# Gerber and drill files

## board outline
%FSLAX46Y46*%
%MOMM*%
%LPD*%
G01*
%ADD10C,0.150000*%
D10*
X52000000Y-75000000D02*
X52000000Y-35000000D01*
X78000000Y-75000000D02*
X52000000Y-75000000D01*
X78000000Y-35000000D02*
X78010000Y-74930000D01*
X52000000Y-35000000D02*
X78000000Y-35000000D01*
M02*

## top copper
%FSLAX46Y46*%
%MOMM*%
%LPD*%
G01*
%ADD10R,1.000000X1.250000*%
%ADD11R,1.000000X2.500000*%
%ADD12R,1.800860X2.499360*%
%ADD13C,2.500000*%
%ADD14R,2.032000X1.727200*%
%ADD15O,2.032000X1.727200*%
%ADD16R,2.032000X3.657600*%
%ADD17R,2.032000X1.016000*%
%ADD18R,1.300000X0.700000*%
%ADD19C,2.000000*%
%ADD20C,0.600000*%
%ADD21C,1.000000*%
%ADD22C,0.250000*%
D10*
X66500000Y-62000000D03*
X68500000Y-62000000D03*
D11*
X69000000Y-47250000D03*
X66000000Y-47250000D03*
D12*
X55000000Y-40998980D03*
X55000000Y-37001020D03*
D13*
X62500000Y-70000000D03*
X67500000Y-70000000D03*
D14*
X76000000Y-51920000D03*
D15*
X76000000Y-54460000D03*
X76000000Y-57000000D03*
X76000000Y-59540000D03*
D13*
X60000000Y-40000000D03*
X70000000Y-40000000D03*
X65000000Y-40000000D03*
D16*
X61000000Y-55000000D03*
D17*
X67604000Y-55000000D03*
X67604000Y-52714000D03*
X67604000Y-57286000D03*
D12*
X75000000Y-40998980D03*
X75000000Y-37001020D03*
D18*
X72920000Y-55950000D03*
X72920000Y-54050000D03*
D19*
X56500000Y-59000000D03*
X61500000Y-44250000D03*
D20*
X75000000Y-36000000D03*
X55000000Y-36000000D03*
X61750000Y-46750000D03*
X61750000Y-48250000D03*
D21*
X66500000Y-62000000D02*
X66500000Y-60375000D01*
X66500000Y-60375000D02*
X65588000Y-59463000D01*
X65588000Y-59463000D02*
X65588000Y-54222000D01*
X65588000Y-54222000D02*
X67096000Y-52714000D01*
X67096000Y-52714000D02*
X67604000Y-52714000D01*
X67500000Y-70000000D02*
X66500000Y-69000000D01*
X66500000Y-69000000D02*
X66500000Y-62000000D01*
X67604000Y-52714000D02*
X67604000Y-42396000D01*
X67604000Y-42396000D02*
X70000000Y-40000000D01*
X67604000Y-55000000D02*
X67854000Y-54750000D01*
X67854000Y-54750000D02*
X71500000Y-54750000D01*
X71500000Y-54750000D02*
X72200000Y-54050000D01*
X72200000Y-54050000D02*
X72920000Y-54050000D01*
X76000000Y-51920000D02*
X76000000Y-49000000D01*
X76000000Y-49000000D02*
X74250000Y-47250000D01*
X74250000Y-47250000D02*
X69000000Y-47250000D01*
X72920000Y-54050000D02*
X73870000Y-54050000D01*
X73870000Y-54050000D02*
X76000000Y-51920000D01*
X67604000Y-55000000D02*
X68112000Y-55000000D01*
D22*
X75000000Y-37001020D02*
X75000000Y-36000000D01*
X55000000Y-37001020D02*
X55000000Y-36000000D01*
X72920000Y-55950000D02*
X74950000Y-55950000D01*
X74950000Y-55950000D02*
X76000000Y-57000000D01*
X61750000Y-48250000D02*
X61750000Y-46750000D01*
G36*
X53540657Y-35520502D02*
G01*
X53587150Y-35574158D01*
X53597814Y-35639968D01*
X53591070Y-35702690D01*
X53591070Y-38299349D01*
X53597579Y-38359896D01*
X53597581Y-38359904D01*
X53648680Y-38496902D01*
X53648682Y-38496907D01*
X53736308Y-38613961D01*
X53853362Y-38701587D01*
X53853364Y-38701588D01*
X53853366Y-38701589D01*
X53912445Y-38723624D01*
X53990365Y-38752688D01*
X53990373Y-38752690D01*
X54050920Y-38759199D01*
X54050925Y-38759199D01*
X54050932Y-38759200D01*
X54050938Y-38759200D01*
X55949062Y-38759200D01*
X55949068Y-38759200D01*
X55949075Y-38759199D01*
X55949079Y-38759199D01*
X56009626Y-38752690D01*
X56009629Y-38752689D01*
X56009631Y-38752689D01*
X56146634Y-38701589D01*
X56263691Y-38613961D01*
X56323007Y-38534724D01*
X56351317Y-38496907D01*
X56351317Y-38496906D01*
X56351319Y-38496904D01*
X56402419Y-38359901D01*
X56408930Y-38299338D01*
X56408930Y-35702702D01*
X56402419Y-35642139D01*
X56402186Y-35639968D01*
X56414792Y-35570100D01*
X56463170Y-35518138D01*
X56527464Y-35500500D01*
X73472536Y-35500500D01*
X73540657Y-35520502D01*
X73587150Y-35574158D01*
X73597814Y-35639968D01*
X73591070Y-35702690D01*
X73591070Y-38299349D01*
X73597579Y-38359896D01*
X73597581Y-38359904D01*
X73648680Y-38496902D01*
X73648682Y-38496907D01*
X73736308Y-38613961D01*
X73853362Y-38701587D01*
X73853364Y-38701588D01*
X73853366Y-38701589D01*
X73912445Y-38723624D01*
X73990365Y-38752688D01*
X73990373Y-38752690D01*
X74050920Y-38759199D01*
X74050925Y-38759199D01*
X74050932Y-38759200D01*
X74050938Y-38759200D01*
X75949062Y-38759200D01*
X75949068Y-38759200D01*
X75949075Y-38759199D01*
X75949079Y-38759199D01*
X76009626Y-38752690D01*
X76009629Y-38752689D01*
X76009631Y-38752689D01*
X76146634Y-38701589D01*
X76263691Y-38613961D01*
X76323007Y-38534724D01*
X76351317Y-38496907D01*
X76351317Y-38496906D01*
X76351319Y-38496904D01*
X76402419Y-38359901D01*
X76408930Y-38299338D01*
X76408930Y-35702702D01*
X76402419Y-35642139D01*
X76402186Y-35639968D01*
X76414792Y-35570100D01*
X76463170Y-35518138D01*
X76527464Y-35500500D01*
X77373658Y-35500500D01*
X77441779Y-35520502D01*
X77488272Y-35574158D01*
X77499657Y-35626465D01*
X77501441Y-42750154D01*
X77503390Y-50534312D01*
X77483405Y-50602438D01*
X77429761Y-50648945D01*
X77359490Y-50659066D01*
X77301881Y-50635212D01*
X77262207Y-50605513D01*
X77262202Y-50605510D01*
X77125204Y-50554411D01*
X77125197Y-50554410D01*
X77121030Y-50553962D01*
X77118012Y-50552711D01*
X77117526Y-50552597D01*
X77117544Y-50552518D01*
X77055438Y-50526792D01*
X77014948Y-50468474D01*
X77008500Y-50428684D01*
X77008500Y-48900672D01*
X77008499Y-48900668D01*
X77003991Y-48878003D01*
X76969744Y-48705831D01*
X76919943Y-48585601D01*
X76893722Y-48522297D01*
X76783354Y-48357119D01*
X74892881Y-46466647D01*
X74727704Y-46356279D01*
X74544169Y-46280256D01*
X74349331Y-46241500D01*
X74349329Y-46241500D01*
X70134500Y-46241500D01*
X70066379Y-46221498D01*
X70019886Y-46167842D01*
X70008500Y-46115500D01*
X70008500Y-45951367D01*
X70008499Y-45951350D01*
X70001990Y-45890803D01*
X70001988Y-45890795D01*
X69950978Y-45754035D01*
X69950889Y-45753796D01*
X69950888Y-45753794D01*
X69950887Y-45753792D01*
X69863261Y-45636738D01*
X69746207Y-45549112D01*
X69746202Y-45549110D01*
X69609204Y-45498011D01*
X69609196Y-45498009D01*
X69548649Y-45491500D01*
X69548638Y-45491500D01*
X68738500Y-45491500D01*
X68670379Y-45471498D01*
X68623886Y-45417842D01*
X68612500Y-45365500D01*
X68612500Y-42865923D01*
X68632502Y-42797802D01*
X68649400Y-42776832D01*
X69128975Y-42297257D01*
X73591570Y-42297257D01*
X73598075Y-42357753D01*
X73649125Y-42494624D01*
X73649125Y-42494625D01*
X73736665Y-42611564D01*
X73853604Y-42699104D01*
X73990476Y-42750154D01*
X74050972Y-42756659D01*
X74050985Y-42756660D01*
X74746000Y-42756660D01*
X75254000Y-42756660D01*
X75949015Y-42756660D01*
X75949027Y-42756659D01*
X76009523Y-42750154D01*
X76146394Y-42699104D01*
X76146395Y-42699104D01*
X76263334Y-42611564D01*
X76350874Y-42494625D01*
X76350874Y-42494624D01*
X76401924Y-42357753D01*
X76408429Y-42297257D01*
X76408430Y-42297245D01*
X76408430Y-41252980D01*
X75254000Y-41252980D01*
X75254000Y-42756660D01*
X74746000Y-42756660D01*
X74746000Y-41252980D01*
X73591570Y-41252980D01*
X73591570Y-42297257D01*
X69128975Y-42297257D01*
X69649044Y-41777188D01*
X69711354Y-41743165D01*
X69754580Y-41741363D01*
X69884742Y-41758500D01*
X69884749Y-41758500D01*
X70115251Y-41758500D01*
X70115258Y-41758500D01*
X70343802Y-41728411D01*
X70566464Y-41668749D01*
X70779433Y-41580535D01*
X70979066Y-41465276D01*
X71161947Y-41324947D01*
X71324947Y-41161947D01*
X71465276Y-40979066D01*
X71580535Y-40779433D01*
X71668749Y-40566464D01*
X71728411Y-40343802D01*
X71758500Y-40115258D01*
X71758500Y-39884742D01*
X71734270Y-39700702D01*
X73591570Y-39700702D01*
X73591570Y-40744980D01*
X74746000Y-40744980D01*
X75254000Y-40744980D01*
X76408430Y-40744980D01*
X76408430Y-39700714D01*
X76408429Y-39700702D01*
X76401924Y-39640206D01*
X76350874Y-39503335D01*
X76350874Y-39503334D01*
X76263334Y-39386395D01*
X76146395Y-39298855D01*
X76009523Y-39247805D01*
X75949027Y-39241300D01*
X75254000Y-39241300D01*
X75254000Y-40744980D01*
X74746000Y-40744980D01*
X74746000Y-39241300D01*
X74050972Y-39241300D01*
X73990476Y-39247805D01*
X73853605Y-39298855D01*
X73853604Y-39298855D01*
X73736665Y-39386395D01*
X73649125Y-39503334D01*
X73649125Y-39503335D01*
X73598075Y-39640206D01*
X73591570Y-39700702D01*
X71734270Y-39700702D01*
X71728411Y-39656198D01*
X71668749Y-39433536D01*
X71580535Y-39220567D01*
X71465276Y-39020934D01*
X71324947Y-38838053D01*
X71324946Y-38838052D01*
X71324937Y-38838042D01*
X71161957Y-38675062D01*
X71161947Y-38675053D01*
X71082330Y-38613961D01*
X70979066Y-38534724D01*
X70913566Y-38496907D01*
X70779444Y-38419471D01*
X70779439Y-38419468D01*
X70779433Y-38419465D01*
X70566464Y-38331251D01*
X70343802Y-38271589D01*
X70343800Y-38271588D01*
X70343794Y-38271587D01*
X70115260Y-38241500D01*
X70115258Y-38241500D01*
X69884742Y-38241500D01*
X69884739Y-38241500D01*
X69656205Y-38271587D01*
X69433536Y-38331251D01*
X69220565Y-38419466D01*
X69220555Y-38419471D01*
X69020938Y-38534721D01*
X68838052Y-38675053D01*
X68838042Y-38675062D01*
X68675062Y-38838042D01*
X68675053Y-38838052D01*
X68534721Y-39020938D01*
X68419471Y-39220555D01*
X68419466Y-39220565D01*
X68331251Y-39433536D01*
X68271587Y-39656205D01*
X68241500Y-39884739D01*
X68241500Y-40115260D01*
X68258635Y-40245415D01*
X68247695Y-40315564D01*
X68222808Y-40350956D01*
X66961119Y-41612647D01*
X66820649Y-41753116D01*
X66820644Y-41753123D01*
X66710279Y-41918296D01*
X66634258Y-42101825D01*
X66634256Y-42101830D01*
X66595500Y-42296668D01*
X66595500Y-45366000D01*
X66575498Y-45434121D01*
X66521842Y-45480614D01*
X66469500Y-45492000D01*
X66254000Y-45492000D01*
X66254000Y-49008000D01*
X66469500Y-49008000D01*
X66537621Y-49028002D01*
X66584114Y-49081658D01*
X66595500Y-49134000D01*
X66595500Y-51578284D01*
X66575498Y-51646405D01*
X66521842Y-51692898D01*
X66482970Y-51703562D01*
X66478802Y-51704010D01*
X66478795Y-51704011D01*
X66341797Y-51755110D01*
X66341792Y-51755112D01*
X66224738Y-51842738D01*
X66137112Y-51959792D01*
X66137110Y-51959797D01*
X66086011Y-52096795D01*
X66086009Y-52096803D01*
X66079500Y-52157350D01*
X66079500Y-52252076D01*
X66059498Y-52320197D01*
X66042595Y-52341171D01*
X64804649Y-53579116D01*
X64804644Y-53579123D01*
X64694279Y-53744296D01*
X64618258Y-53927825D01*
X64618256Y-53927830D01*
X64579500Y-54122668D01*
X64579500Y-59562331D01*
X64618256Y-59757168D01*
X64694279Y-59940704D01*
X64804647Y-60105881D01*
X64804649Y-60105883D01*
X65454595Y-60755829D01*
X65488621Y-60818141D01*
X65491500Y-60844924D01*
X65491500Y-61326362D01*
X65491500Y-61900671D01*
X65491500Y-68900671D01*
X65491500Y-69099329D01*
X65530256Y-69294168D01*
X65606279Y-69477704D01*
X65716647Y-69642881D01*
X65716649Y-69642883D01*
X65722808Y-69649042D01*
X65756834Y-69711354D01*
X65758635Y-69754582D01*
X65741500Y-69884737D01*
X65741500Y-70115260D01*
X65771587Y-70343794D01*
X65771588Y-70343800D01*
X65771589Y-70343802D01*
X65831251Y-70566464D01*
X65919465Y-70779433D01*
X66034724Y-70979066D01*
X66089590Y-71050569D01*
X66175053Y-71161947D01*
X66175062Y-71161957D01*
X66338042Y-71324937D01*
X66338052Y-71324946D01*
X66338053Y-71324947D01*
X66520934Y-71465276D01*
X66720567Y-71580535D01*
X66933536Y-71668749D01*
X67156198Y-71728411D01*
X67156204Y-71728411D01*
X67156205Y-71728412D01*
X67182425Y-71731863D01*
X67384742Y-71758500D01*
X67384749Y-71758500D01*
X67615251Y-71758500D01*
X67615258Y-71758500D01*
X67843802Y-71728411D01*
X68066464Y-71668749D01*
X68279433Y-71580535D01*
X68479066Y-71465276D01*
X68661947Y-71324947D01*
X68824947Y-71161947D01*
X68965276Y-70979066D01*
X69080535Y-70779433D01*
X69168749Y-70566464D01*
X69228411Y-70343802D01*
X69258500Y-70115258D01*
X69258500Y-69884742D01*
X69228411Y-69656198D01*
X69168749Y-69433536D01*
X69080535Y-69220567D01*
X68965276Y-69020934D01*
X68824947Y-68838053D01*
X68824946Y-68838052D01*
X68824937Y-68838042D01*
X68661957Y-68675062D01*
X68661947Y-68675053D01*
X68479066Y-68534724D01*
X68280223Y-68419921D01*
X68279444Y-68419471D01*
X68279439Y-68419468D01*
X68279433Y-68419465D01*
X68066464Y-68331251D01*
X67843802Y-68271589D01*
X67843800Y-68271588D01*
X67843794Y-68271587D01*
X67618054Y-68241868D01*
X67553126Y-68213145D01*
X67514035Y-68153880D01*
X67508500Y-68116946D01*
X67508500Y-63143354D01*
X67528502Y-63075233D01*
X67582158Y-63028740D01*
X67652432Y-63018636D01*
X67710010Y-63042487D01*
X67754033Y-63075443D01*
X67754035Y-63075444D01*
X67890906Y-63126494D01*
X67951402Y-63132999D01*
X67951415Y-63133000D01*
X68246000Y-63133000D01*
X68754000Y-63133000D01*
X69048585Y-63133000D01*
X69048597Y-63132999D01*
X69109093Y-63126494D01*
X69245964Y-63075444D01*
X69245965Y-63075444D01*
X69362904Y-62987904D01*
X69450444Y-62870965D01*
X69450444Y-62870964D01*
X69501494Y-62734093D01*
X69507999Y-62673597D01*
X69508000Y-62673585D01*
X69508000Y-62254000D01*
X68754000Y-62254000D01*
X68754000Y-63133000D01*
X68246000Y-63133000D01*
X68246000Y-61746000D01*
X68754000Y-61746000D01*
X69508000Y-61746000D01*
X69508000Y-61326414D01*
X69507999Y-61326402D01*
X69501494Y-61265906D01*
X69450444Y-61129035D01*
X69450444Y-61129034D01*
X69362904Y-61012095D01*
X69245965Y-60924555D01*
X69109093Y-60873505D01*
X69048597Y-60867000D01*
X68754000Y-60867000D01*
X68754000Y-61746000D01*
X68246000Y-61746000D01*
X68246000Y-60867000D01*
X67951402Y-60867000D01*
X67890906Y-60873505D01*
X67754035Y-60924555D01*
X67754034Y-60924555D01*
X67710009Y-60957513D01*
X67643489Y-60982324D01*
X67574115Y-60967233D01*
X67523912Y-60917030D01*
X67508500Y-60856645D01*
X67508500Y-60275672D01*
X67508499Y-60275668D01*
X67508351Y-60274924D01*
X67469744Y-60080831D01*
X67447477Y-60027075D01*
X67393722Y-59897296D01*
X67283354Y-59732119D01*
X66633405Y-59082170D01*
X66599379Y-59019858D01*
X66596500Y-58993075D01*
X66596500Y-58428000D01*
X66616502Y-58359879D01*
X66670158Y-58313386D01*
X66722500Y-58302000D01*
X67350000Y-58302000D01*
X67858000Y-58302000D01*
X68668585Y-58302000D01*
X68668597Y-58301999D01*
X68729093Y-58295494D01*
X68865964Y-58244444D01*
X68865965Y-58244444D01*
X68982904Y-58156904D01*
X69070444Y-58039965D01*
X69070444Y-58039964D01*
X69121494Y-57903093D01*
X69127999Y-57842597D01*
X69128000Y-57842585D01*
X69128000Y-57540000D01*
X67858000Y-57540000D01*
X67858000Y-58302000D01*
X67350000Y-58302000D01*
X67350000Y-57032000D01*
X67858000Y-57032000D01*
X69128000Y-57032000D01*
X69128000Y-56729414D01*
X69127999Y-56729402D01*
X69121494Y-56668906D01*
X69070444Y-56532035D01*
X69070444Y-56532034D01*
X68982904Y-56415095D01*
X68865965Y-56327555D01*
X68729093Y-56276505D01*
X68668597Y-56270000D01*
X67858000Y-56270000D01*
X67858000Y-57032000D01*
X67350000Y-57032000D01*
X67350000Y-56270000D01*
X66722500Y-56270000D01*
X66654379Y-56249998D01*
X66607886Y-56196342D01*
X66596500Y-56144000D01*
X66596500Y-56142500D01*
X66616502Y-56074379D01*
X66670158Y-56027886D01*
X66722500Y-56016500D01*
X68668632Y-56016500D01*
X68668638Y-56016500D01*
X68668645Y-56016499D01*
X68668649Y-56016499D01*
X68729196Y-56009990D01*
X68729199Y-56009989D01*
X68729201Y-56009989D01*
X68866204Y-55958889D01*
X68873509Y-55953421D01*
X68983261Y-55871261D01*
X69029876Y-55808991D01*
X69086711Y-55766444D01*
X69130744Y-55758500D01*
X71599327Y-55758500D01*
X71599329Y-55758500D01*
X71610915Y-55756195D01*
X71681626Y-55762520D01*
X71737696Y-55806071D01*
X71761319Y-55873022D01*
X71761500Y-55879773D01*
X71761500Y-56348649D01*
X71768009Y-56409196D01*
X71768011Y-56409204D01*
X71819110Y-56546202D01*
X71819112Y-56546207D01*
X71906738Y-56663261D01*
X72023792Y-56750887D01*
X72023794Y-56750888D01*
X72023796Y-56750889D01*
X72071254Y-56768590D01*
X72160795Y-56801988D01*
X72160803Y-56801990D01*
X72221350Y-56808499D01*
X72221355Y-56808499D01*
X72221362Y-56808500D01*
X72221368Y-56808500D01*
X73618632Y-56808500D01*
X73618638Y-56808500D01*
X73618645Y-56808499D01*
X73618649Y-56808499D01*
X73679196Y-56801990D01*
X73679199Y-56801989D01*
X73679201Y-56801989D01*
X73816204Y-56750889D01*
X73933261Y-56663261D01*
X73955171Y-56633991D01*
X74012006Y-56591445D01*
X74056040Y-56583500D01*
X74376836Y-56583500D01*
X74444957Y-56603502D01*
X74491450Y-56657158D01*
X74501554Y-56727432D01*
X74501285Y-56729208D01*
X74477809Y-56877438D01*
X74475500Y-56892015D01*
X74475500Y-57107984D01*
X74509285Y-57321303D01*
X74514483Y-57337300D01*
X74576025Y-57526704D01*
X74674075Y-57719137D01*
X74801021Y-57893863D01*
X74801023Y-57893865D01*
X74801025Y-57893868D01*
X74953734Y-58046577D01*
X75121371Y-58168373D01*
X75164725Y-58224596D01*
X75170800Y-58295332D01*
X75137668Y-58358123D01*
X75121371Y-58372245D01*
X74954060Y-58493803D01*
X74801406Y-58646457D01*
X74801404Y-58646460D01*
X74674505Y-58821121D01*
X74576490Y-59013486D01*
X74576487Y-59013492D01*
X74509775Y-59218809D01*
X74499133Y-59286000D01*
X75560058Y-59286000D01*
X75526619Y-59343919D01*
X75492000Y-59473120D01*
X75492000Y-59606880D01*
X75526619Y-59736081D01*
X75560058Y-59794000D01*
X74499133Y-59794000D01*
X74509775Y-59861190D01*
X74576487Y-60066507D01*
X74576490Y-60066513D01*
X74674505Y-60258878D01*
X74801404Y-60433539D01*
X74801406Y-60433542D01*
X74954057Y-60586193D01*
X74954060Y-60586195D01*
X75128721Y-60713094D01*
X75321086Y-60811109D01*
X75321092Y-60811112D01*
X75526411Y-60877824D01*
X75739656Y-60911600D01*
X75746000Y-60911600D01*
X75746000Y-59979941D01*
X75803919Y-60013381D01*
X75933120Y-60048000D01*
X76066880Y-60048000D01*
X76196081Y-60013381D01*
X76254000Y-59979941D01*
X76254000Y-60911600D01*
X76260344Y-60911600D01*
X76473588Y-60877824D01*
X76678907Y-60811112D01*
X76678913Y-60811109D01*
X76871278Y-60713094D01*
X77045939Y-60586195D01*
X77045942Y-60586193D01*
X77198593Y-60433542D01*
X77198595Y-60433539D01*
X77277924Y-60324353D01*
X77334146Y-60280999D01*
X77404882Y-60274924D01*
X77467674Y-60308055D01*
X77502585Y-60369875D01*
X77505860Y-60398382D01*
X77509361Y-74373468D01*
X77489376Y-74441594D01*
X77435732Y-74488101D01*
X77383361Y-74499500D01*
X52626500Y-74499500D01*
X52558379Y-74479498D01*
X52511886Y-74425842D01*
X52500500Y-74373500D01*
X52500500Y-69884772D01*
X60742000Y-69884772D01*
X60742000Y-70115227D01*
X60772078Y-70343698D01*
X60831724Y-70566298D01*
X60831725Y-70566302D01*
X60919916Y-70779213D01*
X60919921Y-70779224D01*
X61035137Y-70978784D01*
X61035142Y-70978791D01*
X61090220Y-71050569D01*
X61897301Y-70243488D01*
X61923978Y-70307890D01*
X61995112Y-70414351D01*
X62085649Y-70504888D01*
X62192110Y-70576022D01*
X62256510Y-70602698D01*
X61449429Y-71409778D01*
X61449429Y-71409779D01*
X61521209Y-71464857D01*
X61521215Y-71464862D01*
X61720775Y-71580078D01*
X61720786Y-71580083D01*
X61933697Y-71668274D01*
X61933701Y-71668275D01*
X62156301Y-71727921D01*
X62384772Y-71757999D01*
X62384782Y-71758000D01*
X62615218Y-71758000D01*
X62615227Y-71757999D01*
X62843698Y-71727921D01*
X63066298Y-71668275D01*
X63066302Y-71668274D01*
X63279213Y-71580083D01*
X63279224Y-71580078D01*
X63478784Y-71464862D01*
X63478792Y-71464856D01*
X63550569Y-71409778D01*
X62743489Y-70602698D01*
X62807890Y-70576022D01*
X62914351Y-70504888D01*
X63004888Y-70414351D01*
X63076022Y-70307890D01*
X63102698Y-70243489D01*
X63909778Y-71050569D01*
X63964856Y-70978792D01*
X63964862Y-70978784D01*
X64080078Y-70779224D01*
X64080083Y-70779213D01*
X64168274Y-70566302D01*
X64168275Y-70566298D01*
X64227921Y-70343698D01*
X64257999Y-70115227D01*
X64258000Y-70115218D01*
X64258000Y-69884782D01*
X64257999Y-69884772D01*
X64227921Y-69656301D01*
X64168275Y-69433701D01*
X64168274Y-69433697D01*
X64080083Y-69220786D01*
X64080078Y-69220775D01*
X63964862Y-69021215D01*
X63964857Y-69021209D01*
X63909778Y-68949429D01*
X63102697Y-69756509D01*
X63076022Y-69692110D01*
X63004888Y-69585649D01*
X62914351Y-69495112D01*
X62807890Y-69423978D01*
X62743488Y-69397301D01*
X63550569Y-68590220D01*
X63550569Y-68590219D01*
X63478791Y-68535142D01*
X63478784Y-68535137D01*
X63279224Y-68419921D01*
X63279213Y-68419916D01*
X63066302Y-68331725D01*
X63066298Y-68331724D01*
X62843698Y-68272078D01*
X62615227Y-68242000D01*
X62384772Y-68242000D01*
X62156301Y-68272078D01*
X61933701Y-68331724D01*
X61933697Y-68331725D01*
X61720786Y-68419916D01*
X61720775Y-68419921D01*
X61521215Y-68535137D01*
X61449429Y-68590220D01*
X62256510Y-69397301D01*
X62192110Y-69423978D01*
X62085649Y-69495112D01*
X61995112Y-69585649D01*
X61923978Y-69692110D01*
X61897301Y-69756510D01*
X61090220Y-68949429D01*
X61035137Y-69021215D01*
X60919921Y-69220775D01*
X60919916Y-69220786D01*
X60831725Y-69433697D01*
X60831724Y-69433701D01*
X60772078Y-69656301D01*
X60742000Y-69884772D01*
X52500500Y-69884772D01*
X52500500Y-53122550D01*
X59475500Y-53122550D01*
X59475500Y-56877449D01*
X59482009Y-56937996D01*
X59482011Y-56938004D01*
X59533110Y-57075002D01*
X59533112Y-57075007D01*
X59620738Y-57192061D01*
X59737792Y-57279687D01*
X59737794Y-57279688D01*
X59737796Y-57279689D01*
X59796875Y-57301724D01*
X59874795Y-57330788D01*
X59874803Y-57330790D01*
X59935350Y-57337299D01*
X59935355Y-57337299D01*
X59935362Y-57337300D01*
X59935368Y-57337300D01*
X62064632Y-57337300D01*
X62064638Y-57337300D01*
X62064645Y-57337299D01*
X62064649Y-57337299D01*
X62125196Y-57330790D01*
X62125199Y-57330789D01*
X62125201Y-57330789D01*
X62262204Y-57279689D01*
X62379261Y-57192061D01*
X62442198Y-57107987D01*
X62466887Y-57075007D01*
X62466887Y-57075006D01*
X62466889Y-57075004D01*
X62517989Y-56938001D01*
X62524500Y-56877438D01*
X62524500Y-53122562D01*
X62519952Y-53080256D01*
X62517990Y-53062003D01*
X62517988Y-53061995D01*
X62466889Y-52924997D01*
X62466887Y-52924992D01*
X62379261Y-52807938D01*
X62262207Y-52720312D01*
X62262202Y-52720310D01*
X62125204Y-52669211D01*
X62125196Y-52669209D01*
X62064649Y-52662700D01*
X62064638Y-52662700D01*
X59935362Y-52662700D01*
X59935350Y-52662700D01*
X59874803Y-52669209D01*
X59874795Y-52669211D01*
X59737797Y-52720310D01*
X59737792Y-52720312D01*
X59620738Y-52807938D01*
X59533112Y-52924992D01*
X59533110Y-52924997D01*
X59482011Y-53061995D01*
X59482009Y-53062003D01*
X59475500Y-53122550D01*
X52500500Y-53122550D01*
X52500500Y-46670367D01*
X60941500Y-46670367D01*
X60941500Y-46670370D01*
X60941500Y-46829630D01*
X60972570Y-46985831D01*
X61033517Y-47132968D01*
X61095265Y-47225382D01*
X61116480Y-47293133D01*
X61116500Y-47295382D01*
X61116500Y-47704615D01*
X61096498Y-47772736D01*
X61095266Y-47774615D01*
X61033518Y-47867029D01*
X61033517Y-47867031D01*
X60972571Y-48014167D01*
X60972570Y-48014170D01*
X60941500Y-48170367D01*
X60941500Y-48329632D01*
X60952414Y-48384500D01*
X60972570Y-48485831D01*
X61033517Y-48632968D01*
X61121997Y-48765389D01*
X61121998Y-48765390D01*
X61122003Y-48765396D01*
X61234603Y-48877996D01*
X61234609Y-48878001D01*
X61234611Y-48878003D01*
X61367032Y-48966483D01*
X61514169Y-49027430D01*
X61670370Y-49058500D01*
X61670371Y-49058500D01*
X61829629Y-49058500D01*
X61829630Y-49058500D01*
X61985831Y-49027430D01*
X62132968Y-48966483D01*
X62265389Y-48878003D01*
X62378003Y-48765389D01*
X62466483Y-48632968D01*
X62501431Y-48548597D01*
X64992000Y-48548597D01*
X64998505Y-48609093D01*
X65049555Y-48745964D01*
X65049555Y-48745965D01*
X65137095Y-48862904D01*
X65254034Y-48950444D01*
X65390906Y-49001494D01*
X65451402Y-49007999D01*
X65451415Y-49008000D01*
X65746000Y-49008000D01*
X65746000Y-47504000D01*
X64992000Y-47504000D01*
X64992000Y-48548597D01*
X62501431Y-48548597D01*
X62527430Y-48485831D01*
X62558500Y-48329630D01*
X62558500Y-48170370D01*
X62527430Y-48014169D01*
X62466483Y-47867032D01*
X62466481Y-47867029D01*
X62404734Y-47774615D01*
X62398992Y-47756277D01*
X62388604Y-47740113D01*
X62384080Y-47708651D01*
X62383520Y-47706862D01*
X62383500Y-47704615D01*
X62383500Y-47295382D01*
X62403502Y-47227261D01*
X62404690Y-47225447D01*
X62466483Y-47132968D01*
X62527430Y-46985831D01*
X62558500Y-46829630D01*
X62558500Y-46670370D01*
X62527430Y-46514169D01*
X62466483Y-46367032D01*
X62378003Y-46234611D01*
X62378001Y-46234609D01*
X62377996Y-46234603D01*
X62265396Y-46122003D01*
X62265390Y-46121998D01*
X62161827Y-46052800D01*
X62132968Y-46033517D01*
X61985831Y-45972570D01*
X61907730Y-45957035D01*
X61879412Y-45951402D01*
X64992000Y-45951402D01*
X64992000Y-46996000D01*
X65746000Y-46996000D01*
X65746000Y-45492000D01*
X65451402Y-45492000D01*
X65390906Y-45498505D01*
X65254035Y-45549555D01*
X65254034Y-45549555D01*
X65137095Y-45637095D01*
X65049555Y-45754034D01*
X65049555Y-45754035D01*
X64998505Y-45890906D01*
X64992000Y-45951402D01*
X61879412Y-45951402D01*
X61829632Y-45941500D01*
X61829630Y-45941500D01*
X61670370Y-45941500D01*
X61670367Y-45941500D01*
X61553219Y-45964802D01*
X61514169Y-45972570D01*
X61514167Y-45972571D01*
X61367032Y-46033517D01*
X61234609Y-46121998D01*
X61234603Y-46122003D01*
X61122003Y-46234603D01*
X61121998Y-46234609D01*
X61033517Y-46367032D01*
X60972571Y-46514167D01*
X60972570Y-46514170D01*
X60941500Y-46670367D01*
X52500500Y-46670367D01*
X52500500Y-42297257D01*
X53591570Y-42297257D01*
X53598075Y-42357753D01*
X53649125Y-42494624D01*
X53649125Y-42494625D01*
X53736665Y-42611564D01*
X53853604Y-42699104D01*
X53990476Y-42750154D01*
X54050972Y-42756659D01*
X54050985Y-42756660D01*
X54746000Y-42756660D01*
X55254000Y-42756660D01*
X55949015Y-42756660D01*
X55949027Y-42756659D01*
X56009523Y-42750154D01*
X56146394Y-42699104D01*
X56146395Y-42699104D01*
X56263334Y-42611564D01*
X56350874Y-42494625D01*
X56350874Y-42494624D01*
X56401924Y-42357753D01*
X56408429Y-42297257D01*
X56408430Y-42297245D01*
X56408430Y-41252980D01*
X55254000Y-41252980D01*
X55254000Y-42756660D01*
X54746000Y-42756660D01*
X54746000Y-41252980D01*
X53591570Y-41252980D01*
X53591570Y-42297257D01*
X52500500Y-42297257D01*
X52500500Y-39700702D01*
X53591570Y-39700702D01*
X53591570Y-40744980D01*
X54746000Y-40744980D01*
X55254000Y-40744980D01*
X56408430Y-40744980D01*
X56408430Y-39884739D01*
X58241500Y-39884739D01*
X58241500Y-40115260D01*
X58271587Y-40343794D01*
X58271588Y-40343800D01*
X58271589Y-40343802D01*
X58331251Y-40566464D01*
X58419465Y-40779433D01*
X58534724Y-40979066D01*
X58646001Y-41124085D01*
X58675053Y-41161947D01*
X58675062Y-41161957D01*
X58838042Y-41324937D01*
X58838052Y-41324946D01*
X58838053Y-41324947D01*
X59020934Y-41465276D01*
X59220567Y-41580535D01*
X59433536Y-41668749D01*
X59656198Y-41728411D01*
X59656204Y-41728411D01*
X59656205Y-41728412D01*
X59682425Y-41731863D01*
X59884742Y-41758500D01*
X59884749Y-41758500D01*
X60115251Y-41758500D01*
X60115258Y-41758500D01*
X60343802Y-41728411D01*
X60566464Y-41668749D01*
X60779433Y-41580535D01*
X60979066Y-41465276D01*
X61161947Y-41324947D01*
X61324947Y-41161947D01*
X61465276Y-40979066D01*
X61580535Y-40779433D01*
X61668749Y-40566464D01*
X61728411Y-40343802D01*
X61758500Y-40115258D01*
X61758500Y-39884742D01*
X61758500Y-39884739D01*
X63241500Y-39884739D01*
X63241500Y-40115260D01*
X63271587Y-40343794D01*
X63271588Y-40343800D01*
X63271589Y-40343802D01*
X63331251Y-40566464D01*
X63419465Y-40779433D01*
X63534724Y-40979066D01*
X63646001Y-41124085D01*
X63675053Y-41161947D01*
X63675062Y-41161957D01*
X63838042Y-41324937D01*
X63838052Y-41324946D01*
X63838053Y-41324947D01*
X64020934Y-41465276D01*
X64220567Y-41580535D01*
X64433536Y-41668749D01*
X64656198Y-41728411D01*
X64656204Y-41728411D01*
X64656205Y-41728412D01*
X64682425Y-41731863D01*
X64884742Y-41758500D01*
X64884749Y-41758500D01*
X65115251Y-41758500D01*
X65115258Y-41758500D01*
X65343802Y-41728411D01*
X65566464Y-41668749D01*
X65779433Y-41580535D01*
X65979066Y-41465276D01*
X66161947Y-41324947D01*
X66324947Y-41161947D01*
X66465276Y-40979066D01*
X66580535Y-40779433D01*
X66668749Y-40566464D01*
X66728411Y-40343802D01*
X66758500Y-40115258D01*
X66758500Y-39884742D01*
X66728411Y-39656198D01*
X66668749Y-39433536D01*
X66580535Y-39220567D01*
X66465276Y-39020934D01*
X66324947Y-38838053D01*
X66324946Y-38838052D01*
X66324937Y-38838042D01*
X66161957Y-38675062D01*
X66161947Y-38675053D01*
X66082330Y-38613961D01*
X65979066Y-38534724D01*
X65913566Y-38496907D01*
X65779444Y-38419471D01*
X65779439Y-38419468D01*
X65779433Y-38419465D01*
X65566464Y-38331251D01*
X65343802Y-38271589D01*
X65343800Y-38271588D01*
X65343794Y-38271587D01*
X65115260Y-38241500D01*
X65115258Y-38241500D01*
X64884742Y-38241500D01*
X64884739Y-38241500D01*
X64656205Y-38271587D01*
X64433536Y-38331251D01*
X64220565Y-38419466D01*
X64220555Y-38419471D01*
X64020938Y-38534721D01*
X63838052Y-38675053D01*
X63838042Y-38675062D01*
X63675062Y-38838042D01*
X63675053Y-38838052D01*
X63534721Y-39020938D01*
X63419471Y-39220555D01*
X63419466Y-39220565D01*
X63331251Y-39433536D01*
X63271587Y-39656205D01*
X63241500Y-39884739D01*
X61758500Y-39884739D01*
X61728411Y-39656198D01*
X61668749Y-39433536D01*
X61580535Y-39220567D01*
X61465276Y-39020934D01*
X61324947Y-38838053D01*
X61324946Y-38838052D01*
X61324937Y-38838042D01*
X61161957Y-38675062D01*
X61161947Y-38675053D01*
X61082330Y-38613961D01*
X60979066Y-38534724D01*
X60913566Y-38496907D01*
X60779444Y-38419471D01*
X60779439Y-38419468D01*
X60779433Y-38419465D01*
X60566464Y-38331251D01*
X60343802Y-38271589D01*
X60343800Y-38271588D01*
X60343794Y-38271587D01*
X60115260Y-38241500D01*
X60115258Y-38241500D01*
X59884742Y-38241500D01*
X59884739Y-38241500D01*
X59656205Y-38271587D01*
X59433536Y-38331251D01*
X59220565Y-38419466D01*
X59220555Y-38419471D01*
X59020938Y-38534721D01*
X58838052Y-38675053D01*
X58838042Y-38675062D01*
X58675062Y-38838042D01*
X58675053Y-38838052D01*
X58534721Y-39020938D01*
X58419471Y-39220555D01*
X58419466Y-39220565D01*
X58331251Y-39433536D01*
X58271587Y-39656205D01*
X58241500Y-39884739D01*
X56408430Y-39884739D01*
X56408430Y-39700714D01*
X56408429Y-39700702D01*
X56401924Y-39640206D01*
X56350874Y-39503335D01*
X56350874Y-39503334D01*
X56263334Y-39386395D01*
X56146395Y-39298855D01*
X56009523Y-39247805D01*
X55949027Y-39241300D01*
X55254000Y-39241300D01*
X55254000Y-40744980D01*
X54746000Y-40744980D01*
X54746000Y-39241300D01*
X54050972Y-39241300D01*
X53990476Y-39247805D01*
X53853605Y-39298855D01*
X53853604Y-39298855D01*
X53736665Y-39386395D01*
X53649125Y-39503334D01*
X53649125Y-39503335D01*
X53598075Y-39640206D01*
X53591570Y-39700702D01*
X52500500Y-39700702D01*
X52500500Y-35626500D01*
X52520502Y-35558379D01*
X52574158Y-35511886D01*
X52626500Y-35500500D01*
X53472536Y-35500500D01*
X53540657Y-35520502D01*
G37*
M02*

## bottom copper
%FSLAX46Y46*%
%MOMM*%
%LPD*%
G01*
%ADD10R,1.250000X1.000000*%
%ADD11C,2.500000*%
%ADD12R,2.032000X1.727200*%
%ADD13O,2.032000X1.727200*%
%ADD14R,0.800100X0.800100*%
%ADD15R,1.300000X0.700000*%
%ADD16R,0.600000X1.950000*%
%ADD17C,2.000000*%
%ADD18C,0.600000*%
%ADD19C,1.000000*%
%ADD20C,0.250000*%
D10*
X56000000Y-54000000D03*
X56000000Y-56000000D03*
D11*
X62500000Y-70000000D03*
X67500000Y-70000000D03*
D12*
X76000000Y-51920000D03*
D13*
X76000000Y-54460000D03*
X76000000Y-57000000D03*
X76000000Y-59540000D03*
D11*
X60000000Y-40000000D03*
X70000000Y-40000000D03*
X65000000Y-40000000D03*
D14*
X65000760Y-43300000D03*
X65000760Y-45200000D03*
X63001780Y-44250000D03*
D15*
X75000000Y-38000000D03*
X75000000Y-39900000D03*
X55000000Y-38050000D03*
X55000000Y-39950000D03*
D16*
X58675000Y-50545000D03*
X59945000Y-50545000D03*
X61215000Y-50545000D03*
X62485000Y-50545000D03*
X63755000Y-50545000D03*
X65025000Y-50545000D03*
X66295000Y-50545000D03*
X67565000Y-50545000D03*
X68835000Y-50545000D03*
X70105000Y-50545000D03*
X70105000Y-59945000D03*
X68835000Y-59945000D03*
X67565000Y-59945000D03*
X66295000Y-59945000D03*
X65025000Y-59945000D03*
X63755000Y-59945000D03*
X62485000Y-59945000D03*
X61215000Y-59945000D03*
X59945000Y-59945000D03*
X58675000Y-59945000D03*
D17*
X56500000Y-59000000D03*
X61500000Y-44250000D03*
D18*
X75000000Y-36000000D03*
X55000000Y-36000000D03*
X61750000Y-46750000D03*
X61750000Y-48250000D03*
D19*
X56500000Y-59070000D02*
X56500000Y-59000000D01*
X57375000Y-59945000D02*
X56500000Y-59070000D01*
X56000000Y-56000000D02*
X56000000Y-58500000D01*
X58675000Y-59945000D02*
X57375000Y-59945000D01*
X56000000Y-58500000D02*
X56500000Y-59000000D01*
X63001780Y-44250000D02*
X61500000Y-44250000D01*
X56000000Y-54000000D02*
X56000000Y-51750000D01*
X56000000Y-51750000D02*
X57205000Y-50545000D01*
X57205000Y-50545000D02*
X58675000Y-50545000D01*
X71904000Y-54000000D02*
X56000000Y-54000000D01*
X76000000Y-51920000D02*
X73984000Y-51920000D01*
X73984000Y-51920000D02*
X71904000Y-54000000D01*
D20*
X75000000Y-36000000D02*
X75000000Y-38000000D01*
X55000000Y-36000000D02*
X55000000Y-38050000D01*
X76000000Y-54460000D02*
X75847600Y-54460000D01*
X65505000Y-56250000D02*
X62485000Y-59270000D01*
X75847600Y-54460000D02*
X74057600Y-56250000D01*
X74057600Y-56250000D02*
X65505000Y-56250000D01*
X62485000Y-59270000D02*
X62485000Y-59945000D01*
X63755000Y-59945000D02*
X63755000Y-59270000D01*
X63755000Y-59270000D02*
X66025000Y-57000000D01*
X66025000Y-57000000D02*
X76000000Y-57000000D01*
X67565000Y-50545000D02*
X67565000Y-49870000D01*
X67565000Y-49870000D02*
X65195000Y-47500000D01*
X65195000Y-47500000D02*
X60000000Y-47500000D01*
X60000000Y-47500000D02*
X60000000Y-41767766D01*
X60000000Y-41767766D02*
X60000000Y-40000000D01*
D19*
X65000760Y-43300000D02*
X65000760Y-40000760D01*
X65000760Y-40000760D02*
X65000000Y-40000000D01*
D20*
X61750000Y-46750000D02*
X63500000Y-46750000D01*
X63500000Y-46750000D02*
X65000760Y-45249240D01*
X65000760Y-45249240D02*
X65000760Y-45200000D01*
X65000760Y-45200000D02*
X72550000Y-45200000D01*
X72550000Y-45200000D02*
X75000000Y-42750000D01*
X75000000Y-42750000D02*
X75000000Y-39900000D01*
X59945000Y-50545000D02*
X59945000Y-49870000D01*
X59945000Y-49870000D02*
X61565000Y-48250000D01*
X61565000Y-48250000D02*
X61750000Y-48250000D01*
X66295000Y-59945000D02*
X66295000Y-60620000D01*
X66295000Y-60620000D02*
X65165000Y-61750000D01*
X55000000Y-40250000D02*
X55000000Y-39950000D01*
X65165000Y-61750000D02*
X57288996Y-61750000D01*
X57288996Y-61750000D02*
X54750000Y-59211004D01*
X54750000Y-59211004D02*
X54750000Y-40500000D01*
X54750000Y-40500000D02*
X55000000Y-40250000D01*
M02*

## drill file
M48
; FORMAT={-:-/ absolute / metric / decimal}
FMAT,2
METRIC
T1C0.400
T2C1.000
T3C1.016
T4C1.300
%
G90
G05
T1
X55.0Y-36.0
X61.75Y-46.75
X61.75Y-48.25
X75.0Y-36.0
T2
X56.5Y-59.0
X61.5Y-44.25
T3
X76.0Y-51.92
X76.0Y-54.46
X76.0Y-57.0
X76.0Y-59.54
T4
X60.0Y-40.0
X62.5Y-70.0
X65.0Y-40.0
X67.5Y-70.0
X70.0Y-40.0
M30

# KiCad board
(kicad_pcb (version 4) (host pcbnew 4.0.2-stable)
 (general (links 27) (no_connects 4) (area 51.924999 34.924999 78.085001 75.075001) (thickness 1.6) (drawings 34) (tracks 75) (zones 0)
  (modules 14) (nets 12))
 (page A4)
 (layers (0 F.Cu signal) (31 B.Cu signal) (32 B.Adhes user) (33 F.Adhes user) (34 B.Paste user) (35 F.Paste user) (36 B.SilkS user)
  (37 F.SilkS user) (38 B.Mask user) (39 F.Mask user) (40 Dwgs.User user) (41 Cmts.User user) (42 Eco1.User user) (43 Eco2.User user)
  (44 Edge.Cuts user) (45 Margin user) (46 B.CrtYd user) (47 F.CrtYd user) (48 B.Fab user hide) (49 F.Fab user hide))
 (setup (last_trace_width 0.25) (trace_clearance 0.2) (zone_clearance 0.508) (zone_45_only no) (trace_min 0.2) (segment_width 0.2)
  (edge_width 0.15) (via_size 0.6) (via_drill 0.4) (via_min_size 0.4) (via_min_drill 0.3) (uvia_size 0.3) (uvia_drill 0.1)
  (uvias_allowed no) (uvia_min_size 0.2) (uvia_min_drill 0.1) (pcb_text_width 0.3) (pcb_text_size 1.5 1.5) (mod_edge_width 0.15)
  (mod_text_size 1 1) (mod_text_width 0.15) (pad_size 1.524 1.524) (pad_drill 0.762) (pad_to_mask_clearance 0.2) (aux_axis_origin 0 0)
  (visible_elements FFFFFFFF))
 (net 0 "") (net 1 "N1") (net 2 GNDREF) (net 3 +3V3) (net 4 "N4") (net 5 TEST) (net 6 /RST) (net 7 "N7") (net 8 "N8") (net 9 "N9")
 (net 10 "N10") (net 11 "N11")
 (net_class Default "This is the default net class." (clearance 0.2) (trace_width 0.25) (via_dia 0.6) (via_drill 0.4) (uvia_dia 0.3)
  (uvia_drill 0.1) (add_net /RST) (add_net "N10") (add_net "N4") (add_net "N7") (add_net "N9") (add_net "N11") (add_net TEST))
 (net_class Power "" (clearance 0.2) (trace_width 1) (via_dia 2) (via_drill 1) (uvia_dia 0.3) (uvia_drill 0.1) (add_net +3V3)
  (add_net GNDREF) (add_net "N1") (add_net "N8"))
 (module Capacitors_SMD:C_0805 (layer F.Cu) (at 67.5 62)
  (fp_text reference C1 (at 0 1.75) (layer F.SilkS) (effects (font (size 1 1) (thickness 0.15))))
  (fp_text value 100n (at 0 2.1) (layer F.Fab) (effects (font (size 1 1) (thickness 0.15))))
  (pad 1 smd rect (at -1 0) (size 1 1.25) (layers F.Cu F.Paste F.Mask) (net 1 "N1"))
  (pad 2 smd rect (at 1 0) (size 1 1.25) (layers F.Cu F.Paste F.Mask) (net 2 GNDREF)))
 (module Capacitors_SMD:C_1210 (layer F.Cu) (at 67.5 47.25 180)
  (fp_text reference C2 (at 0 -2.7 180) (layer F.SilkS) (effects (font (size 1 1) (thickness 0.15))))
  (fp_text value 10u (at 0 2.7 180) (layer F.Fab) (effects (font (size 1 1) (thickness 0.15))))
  (pad 1 smd rect (at -1.5 0 180) (size 1 2.5) (layers F.Cu F.Paste F.Mask) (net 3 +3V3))
  (pad 2 smd rect (at 1.5 0 180) (size 1 2.5) (layers F.Cu F.Paste F.Mask) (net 2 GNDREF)))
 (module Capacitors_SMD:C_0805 (layer B.Cu) (at 56 55 270)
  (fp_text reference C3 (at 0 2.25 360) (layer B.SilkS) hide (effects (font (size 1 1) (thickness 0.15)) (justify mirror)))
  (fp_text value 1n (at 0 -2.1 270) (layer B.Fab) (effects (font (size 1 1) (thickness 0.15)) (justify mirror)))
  (pad 1 smd rect (at -1 0 270) (size 1 1.25) (layers B.Cu B.Paste B.Mask) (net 3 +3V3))
  (pad 2 smd rect (at 1 0 270) (size 1 1.25) (layers B.Cu B.Paste B.Mask) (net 2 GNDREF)))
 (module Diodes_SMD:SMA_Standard (layer F.Cu) (at 55 39 90)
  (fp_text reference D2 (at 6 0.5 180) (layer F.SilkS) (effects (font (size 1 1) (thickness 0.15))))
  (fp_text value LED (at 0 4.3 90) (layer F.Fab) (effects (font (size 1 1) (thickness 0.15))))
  (pad 1 smd rect (at -1.99898 0 90) (size 2.49936 1.80086) (layers F.Cu F.Paste F.Mask) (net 2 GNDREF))
  (pad 2 smd rect (at 1.99898 0 90) (size 2.49936 1.80086) (layers F.Cu F.Paste F.Mask) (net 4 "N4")))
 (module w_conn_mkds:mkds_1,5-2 (layer F.Cu) (at 65 70)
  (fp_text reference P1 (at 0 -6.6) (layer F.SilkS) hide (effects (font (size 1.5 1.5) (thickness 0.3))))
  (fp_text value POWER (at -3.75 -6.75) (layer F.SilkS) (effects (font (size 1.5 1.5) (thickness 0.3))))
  (pad 1 thru_hole circle (at -2.5 0) (size 2.5 2.5) (drill 1.3) (layers *.Cu *.Mask F.SilkS) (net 2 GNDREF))
  (pad 2 thru_hole circle (at 2.5 0) (size 2.5 2.5) (drill 1.3) (layers *.Cu *.Mask F.SilkS) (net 1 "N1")))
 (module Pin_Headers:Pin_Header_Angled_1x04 (layer F.Cu) (at 76 51.92)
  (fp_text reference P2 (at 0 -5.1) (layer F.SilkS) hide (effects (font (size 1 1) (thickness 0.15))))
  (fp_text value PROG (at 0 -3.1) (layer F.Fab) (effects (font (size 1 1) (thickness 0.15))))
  (pad 1 thru_hole rect (at 0 0) (size 2.032 1.7272) (drill 1.016) (layers *.Cu *.Mask F.SilkS) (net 3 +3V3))
  (pad 2 thru_hole oval (at 0 2.54) (size 2.032 1.7272) (drill 1.016) (layers *.Cu *.Mask F.SilkS) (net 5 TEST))
  (pad 3 thru_hole oval (at 0 5.08) (size 2.032 1.7272) (drill 1.016) (layers *.Cu *.Mask F.SilkS) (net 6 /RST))
  (pad 4 thru_hole oval (at 0 7.62) (size 2.032 1.7272) (drill 1.016) (layers *.Cu *.Mask F.SilkS) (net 2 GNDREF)))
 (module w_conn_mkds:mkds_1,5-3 (layer F.Cu) (at 65 40 180)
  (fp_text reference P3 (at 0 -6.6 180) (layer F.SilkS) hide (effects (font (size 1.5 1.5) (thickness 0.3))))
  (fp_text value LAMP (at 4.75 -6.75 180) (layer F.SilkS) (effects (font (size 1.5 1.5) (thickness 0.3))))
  (pad 3 thru_hole circle (at 5 0 180) (size 2.5 2.5) (drill 1.3) (layers *.Cu *.Mask F.SilkS) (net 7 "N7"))
  (pad 1 thru_hole circle (at -5 0 180) (size 2.5 2.5) (drill 1.3) (layers *.Cu *.Mask F.SilkS) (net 1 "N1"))
  (pad 2 thru_hole circle (at 0 0 180) (size 2.5 2.5) (drill 1.3) (layers *.Cu *.Mask F.SilkS) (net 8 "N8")))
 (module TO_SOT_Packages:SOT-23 (layer B.Cu) (at 64 44.25 270)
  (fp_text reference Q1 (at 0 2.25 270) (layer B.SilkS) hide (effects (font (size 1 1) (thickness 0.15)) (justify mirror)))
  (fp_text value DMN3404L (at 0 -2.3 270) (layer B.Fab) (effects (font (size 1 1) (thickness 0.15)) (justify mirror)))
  (pad 1 smd rect (at -0.95 -1.00076 270) (size 0.8001 0.8001) (layers B.Cu B.Paste B.Mask) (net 8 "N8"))
  (pad 2 smd rect (at 0.95 -1.00076 270) (size 0.8001 0.8001) (layers B.Cu B.Paste B.Mask) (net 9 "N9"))
  (pad 3 smd rect (at 0 0.99822 270) (size 0.8001 0.8001) (layers B.Cu B.Paste B.Mask) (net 2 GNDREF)))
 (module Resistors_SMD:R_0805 (layer B.Cu) (at 75 38.95 270)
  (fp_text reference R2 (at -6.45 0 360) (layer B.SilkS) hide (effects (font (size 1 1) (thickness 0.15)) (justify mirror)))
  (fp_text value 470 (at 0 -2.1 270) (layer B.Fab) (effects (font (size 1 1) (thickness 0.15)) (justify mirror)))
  (pad 1 smd rect (at -0.95 0 270) (size 0.7 1.3) (layers B.Cu B.Paste B.Mask) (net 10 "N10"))
  (pad 2 smd rect (at 0.95 0 270) (size 0.7 1.3) (layers B.Cu B.Paste B.Mask) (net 9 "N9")))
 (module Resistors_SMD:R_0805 (layer B.Cu) (at 55 39 270)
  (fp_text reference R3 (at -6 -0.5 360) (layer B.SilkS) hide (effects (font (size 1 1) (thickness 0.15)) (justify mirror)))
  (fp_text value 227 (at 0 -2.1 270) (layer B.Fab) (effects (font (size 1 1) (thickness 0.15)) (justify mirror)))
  (pad 1 smd rect (at -0.95 0 270) (size 0.7 1.3) (layers B.Cu B.Paste B.Mask) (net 4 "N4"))
  (pad 2 smd rect (at 0.95 0 270) (size 0.7 1.3) (layers B.Cu B.Paste B.Mask) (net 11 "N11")))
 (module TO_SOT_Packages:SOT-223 (layer F.Cu) (at 64.302 55 90)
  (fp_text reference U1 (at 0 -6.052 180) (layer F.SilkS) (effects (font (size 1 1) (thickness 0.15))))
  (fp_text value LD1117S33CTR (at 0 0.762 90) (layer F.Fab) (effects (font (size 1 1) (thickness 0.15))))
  (pad 4 smd rect (at 0 -3.302 90) (size 3.6576 2.032) (layers F.Cu F.Paste F.Mask))
  (pad 2 smd rect (at 0 3.302 90) (size 1.016 2.032) (layers F.Cu F.Paste F.Mask) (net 3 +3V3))
  (pad 3 smd rect (at 2.286 3.302 90) (size 1.016 2.032) (layers F.Cu F.Paste F.Mask) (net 1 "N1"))
  (pad 1 smd rect (at -2.286 3.302 90) (size 1.016 2.032) (layers F.Cu F.Paste F.Mask) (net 2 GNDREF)))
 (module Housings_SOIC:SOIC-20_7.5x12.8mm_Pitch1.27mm (layer B.Cu) (at 64.39 55.245 270)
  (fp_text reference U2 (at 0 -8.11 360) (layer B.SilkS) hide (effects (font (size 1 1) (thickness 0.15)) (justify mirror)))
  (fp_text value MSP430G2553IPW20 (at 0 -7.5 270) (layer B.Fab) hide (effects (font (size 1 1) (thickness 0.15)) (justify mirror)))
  (pad 1 smd rect (at -4.7 5.715 270) (size 1.95 0.6) (layers B.Cu B.Paste B.Mask) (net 3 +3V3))
  (pad 2 smd rect (at -4.7 4.445 270) (size 1.95 0.6) (layers B.Cu B.Paste B.Mask) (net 9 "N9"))
  (pad 3 smd rect (at -4.7 3.175 270) (size 1.95 0.6) (layers B.Cu B.Paste B.Mask))
  (pad 4 smd rect (at -4.7 1.905 270) (size 1.95 0.6) (layers B.Cu B.Paste B.Mask))
  (pad 5 smd rect (at -4.7 0.635 270) (size 1.95 0.6) (layers B.Cu B.Paste B.Mask))
  (pad 6 smd rect (at -4.7 -0.635 270) (size 1.95 0.6) (layers B.Cu B.Paste B.Mask))
  (pad 7 smd rect (at -4.7 -1.905 270) (size 1.95 0.6) (layers B.Cu B.Paste B.Mask))
  (pad 8 smd rect (at -4.7 -3.175 270) (size 1.95 0.6) (layers B.Cu B.Paste B.Mask) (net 7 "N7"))
  (pad 9 smd rect (at -4.7 -4.445 270) (size 1.95 0.6) (layers B.Cu B.Paste B.Mask))
  (pad 10 smd rect (at -4.7 -5.715 270) (size 1.95 0.6) (layers B.Cu B.Paste B.Mask))
  (pad 11 smd rect (at 4.7 -5.715 270) (size 1.95 0.6) (layers B.Cu B.Paste B.Mask))
  (pad 12 smd rect (at 4.7 -4.445 270) (size 1.95 0.6) (layers B.Cu B.Paste B.Mask))
  (pad 13 smd rect (at 4.7 -3.175 270) (size 1.95 0.6) (layers B.Cu B.Paste B.Mask))
  (pad 14 smd rect (at 4.7 -1.905 270) (size 1.95 0.6) (layers B.Cu B.Paste B.Mask) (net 11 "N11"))
  (pad 15 smd rect (at 4.7 -0.635 270) (size 1.95 0.6) (layers B.Cu B.Paste B.Mask))
  (pad 16 smd rect (at 4.7 0.635 270) (size 1.95 0.6) (layers B.Cu B.Paste B.Mask) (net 6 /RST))
  (pad 17 smd rect (at 4.7 1.905 270) (size 1.95 0.6) (layers B.Cu B.Paste B.Mask) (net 5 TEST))
  (pad 18 smd rect (at 4.7 3.175 270) (size 1.95 0.6) (layers B.Cu B.Paste B.Mask))
  (pad 19 smd rect (at 4.7 4.445 270) (size 1.95 0.6) (layers B.Cu B.Paste B.Mask))
  (pad 20 smd rect (at 4.7 5.715 270) (size 1.95 0.6) (layers B.Cu B.Paste B.Mask) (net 2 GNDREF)))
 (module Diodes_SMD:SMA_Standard (layer F.Cu) (at 75 39 90)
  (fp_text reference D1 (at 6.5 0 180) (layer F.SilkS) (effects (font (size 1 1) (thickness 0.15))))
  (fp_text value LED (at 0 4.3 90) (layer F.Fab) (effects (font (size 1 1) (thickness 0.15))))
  (pad 1 smd rect (at -1.99898 0 90) (size 2.49936 1.80086) (layers F.Cu F.Paste F.Mask) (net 2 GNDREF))
  (pad 2 smd rect (at 1.99898 0 90) (size 2.49936 1.80086) (layers F.Cu F.Paste F.Mask) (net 10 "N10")))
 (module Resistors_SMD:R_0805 (layer F.Cu) (at 72.92 55 90)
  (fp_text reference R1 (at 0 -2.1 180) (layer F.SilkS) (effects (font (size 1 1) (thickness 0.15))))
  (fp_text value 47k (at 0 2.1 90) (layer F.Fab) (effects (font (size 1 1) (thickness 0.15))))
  (pad 1 smd rect (at -0.95 0 90) (size 0.7 1.3) (layers F.Cu F.Paste F.Mask) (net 6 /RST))
  (pad 2 smd rect (at 0.95 0 90) (size 0.7 1.3) (layers F.Cu F.Paste F.Mask) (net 3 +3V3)))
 (gr_line (start 52 75) (end 52 35) (layer Edge.Cuts) (width 0.15))
 (gr_line (start 78 75) (end 52 75) (layer Edge.Cuts) (width 0.15))
 (gr_line (start 78 35) (end 78.01 74.93) (layer Edge.Cuts) (width 0.15))
 (gr_line (start 52 35) (end 78 35) (layer Edge.Cuts) (width 0.15))
 (segment (start 66.5 62) (end 66.5 60.375) (width 1) (layer F.Cu) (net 1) (status 10))
 (segment (start 66.5 60.375) (end 65.588 59.463) (width 1) (layer F.Cu) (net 1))
 (segment (start 65.588 59.463) (end 65.588 54.222) (width 1) (layer F.Cu) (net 1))
 (segment (start 65.588 54.222) (end 67.096 52.714) (width 1) (layer F.Cu) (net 1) (status 20))
 (segment (start 67.096 52.714) (end 67.604 52.714) (width 1) (layer F.Cu) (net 1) (status 30))
 (segment (start 67.5 70) (end 66.5 69) (width 1) (layer F.Cu) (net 1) (status 10))
 (segment (start 66.5 69) (end 66.5 62) (width 1) (layer F.Cu) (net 1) (status 20))
 (segment (start 67.604 52.714) (end 67.604 42.396) (width 1) (layer F.Cu) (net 1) (status 10))
 (segment (start 67.604 42.396) (end 70 40) (width 1) (layer F.Cu) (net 1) (status 20))
 (segment (start 56.5 59.07) (end 56.5 59) (width 1) (layer B.Cu) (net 2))
 (segment (start 57.375 59.945) (end 56.5 59.07) (width 1) (layer B.Cu) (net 2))
 (segment (start 56 56) (end 56 58.5) (width 1) (layer B.Cu) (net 2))
 (via (at 56.5 59) (size 2) (drill 1) (layers F.Cu B.Cu) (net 2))
 (segment (start 58.675 59.945) (end 57.375 59.945) (width 1) (layer B.Cu) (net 2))
 (segment (start 56 58.5) (end 56.5 59) (width 1) (layer B.Cu) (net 2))
 (segment (start 63.00178 44.25) (end 61.5 44.25) (width 1) (layer B.Cu) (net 2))
 (via (at 61.5 44.25) (size 2) (drill 1) (layers F.Cu B.Cu) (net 2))
 (segment (start 67.604 55) (end 67.854 54.75) (width 1) (layer F.Cu) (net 3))
 (segment (start 67.854 54.75) (end 71.5 54.75) (width 1) (layer F.Cu) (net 3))
 (segment (start 71.5 54.75) (end 72.2 54.05) (width 1) (layer F.Cu) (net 3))
 (segment (start 72.2 54.05) (end 72.92 54.05) (width 1) (layer F.Cu) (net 3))
 (segment (start 76 51.92) (end 76 49) (width 1) (layer F.Cu) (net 3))
 (segment (start 76 49) (end 74.25 47.25) (width 1) (layer F.Cu) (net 3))
 (segment (start 74.25 47.25) (end 69 47.25) (width 1) (layer F.Cu) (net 3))
 (segment (start 56 54) (end 56 51.75) (width 1) (layer B.Cu) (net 3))
 (segment (start 56 51.75) (end 57.205 50.545) (width 1) (layer B.Cu) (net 3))
 (segment (start 57.205 50.545) (end 58.675 50.545) (width 1) (layer B.Cu) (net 3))
 (segment (start 71.904 54) (end 56 54) (width 1) (layer B.Cu) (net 3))
 (segment (start 76 51.92) (end 73.984 51.92) (width 1) (layer B.Cu) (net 3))
 (segment (start 73.984 51.92) (end 71.904 54) (width 1) (layer B.Cu) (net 3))
 (segment (start 72.92 54.05) (end 73.87 54.05) (width 1) (layer F.Cu) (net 3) (status 10))
 (segment (start 73.87 54.05) (end 76 51.92) (width 1) (layer F.Cu) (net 3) (status 20))
 (segment (start 67.604 55) (end 68.112 55) (width 1) (layer F.Cu) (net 3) (status 30))
 (segment (start 75 36) (end 75 38) (width 0.25) (layer B.Cu) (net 10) (status 20))
 (segment (start 75 37.00102) (end 75 36) (width 0.25) (layer F.Cu) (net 10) (status 30))
 (via (at 75 36) (size 0.6) (drill 0.4) (layers F.Cu B.Cu) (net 10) (status 30))
 (segment (start 55 36) (end 55 38.05) (width 0.25) (layer B.Cu) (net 4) (status 20))
 (segment (start 55 37.00102) (end 55 36) (width 0.25) (layer F.Cu) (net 4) (status 30))
 (via (at 55 36) (size 0.6) (drill 0.4) (layers F.Cu B.Cu) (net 4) (status 30))
 (segment (start 76 54.46) (end 75.8476 54.46) (width 0.25) (layer B.Cu) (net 5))
 (segment (start 65.505 56.25) (end 62.485 59.27) (width 0.25) (layer B.Cu) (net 5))
 (segment (start 75.8476 54.46) (end 74.0576 56.25) (width 0.25) (layer B.Cu) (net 5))
 (segment (start 74.0576 56.25) (end 65.505 56.25) (width 0.25) (layer B.Cu) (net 5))
 (segment (start 62.485 59.27) (end 62.485 59.945) (width 0.25) (layer B.Cu) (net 5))
 (segment (start 72.92 55.95) (end 74.95 55.95) (width 0.25) (layer F.Cu) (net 6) (status 10))
 (segment (start 74.95 55.95) (end 76 57) (width 0.25) (layer F.Cu) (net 6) (status 20))
 (segment (start 63.755 59.945) (end 63.755 59.27) (width 0.25) (layer B.Cu) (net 6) (status 30))
 (segment (start 63.755 59.27) (end 66.025 57) (width 0.25) (layer B.Cu) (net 6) (status 10))
 (segment (start 66.025 57) (end 76 57) (width 0.25) (layer B.Cu) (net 6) (status 20))
 (segment (start 67.565 50.545) (end 67.565 49.87) (width 0.25) (layer B.Cu) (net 7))
 (segment (start 67.565 49.87) (end 65.195 47.5) (width 0.25) (layer B.Cu) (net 7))
 (segment (start 65.195 47.5) (end 60 47.5) (width 0.25) (layer B.Cu) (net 7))
 (segment (start 60 47.5) (end 60 41.767766) (width 0.25) (layer B.Cu) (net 7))
 (segment (start 60 41.767766) (end 60 40) (width 0.25) (layer B.Cu) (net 7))
 (segment (start 65.00076 43.3) (end 65.00076 40.00076) (width 1) (layer B.Cu) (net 8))
 (segment (start 65.00076 40.00076) (end 65 40) (width 1) (layer B.Cu) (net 8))
 (segment (start 61.75 46.75) (end 63.5 46.75) (width 0.25) (layer B.Cu) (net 9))
 (segment (start 63.5 46.75) (end 65.00076 45.24924) (width 0.25) (layer B.Cu) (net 9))
 (segment (start 65.00076 45.24924) (end 65.00076 45.2) (width 0.25) (layer B.Cu) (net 9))
 (segment (start 65.00076 45.2) (end 72.55 45.2) (width 0.25) (layer B.Cu) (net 9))
 (segment (start 72.55 45.2) (end 75 42.75) (width 0.25) (layer B.Cu) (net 9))
 (segment (start 75 42.75) (end 75 39.9) (width 0.25) (layer B.Cu) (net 9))
 (segment (start 61.75 48.25) (end 61.75 46.75) (width 0.25) (layer F.Cu) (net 9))
 (via (at 61.75 46.75) (size 0.6) (drill 0.4) (layers F.Cu B.Cu) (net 9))
 (segment (start 59.945 50.545) (end 59.945 49.87) (width 0.25) (layer B.Cu) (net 9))
 (segment (start 59.945 49.87) (end 61.565 48.25) (width 0.25) (layer B.Cu) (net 9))
 (segment (start 61.565 48.25) (end 61.75 48.25) (width 0.25) (layer B.Cu) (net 9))
 (via (at 61.75 48.25) (size 0.6) (drill 0.4) (layers F.Cu B.Cu) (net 9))
 (segment (start 66.295 59.945) (end 66.295 60.62) (width 0.25) (layer B.Cu) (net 11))
 (segment (start 66.295 60.62) (end 65.165 61.75) (width 0.25) (layer B.Cu) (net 11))
 (segment (start 55 40.25) (end 55 39.95) (width 0.25) (layer B.Cu) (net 11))
 (segment (start 65.165 61.75) (end 57.288996 61.75) (width 0.25) (layer B.Cu) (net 11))
 (segment (start 57.288996 61.75) (end 54.75 59.211004) (width 0.25) (layer B.Cu) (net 11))
 (segment (start 54.75 59.211004) (end 54.75 40.5) (width 0.25) (layer B.Cu) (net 11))
 (segment (start 54.75 40.5) (end 55 40.25) (width 0.25) (layer B.Cu) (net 11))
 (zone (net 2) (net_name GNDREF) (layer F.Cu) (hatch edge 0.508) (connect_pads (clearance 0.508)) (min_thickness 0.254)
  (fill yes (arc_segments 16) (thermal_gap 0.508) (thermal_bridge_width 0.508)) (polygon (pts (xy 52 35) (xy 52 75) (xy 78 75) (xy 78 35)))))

